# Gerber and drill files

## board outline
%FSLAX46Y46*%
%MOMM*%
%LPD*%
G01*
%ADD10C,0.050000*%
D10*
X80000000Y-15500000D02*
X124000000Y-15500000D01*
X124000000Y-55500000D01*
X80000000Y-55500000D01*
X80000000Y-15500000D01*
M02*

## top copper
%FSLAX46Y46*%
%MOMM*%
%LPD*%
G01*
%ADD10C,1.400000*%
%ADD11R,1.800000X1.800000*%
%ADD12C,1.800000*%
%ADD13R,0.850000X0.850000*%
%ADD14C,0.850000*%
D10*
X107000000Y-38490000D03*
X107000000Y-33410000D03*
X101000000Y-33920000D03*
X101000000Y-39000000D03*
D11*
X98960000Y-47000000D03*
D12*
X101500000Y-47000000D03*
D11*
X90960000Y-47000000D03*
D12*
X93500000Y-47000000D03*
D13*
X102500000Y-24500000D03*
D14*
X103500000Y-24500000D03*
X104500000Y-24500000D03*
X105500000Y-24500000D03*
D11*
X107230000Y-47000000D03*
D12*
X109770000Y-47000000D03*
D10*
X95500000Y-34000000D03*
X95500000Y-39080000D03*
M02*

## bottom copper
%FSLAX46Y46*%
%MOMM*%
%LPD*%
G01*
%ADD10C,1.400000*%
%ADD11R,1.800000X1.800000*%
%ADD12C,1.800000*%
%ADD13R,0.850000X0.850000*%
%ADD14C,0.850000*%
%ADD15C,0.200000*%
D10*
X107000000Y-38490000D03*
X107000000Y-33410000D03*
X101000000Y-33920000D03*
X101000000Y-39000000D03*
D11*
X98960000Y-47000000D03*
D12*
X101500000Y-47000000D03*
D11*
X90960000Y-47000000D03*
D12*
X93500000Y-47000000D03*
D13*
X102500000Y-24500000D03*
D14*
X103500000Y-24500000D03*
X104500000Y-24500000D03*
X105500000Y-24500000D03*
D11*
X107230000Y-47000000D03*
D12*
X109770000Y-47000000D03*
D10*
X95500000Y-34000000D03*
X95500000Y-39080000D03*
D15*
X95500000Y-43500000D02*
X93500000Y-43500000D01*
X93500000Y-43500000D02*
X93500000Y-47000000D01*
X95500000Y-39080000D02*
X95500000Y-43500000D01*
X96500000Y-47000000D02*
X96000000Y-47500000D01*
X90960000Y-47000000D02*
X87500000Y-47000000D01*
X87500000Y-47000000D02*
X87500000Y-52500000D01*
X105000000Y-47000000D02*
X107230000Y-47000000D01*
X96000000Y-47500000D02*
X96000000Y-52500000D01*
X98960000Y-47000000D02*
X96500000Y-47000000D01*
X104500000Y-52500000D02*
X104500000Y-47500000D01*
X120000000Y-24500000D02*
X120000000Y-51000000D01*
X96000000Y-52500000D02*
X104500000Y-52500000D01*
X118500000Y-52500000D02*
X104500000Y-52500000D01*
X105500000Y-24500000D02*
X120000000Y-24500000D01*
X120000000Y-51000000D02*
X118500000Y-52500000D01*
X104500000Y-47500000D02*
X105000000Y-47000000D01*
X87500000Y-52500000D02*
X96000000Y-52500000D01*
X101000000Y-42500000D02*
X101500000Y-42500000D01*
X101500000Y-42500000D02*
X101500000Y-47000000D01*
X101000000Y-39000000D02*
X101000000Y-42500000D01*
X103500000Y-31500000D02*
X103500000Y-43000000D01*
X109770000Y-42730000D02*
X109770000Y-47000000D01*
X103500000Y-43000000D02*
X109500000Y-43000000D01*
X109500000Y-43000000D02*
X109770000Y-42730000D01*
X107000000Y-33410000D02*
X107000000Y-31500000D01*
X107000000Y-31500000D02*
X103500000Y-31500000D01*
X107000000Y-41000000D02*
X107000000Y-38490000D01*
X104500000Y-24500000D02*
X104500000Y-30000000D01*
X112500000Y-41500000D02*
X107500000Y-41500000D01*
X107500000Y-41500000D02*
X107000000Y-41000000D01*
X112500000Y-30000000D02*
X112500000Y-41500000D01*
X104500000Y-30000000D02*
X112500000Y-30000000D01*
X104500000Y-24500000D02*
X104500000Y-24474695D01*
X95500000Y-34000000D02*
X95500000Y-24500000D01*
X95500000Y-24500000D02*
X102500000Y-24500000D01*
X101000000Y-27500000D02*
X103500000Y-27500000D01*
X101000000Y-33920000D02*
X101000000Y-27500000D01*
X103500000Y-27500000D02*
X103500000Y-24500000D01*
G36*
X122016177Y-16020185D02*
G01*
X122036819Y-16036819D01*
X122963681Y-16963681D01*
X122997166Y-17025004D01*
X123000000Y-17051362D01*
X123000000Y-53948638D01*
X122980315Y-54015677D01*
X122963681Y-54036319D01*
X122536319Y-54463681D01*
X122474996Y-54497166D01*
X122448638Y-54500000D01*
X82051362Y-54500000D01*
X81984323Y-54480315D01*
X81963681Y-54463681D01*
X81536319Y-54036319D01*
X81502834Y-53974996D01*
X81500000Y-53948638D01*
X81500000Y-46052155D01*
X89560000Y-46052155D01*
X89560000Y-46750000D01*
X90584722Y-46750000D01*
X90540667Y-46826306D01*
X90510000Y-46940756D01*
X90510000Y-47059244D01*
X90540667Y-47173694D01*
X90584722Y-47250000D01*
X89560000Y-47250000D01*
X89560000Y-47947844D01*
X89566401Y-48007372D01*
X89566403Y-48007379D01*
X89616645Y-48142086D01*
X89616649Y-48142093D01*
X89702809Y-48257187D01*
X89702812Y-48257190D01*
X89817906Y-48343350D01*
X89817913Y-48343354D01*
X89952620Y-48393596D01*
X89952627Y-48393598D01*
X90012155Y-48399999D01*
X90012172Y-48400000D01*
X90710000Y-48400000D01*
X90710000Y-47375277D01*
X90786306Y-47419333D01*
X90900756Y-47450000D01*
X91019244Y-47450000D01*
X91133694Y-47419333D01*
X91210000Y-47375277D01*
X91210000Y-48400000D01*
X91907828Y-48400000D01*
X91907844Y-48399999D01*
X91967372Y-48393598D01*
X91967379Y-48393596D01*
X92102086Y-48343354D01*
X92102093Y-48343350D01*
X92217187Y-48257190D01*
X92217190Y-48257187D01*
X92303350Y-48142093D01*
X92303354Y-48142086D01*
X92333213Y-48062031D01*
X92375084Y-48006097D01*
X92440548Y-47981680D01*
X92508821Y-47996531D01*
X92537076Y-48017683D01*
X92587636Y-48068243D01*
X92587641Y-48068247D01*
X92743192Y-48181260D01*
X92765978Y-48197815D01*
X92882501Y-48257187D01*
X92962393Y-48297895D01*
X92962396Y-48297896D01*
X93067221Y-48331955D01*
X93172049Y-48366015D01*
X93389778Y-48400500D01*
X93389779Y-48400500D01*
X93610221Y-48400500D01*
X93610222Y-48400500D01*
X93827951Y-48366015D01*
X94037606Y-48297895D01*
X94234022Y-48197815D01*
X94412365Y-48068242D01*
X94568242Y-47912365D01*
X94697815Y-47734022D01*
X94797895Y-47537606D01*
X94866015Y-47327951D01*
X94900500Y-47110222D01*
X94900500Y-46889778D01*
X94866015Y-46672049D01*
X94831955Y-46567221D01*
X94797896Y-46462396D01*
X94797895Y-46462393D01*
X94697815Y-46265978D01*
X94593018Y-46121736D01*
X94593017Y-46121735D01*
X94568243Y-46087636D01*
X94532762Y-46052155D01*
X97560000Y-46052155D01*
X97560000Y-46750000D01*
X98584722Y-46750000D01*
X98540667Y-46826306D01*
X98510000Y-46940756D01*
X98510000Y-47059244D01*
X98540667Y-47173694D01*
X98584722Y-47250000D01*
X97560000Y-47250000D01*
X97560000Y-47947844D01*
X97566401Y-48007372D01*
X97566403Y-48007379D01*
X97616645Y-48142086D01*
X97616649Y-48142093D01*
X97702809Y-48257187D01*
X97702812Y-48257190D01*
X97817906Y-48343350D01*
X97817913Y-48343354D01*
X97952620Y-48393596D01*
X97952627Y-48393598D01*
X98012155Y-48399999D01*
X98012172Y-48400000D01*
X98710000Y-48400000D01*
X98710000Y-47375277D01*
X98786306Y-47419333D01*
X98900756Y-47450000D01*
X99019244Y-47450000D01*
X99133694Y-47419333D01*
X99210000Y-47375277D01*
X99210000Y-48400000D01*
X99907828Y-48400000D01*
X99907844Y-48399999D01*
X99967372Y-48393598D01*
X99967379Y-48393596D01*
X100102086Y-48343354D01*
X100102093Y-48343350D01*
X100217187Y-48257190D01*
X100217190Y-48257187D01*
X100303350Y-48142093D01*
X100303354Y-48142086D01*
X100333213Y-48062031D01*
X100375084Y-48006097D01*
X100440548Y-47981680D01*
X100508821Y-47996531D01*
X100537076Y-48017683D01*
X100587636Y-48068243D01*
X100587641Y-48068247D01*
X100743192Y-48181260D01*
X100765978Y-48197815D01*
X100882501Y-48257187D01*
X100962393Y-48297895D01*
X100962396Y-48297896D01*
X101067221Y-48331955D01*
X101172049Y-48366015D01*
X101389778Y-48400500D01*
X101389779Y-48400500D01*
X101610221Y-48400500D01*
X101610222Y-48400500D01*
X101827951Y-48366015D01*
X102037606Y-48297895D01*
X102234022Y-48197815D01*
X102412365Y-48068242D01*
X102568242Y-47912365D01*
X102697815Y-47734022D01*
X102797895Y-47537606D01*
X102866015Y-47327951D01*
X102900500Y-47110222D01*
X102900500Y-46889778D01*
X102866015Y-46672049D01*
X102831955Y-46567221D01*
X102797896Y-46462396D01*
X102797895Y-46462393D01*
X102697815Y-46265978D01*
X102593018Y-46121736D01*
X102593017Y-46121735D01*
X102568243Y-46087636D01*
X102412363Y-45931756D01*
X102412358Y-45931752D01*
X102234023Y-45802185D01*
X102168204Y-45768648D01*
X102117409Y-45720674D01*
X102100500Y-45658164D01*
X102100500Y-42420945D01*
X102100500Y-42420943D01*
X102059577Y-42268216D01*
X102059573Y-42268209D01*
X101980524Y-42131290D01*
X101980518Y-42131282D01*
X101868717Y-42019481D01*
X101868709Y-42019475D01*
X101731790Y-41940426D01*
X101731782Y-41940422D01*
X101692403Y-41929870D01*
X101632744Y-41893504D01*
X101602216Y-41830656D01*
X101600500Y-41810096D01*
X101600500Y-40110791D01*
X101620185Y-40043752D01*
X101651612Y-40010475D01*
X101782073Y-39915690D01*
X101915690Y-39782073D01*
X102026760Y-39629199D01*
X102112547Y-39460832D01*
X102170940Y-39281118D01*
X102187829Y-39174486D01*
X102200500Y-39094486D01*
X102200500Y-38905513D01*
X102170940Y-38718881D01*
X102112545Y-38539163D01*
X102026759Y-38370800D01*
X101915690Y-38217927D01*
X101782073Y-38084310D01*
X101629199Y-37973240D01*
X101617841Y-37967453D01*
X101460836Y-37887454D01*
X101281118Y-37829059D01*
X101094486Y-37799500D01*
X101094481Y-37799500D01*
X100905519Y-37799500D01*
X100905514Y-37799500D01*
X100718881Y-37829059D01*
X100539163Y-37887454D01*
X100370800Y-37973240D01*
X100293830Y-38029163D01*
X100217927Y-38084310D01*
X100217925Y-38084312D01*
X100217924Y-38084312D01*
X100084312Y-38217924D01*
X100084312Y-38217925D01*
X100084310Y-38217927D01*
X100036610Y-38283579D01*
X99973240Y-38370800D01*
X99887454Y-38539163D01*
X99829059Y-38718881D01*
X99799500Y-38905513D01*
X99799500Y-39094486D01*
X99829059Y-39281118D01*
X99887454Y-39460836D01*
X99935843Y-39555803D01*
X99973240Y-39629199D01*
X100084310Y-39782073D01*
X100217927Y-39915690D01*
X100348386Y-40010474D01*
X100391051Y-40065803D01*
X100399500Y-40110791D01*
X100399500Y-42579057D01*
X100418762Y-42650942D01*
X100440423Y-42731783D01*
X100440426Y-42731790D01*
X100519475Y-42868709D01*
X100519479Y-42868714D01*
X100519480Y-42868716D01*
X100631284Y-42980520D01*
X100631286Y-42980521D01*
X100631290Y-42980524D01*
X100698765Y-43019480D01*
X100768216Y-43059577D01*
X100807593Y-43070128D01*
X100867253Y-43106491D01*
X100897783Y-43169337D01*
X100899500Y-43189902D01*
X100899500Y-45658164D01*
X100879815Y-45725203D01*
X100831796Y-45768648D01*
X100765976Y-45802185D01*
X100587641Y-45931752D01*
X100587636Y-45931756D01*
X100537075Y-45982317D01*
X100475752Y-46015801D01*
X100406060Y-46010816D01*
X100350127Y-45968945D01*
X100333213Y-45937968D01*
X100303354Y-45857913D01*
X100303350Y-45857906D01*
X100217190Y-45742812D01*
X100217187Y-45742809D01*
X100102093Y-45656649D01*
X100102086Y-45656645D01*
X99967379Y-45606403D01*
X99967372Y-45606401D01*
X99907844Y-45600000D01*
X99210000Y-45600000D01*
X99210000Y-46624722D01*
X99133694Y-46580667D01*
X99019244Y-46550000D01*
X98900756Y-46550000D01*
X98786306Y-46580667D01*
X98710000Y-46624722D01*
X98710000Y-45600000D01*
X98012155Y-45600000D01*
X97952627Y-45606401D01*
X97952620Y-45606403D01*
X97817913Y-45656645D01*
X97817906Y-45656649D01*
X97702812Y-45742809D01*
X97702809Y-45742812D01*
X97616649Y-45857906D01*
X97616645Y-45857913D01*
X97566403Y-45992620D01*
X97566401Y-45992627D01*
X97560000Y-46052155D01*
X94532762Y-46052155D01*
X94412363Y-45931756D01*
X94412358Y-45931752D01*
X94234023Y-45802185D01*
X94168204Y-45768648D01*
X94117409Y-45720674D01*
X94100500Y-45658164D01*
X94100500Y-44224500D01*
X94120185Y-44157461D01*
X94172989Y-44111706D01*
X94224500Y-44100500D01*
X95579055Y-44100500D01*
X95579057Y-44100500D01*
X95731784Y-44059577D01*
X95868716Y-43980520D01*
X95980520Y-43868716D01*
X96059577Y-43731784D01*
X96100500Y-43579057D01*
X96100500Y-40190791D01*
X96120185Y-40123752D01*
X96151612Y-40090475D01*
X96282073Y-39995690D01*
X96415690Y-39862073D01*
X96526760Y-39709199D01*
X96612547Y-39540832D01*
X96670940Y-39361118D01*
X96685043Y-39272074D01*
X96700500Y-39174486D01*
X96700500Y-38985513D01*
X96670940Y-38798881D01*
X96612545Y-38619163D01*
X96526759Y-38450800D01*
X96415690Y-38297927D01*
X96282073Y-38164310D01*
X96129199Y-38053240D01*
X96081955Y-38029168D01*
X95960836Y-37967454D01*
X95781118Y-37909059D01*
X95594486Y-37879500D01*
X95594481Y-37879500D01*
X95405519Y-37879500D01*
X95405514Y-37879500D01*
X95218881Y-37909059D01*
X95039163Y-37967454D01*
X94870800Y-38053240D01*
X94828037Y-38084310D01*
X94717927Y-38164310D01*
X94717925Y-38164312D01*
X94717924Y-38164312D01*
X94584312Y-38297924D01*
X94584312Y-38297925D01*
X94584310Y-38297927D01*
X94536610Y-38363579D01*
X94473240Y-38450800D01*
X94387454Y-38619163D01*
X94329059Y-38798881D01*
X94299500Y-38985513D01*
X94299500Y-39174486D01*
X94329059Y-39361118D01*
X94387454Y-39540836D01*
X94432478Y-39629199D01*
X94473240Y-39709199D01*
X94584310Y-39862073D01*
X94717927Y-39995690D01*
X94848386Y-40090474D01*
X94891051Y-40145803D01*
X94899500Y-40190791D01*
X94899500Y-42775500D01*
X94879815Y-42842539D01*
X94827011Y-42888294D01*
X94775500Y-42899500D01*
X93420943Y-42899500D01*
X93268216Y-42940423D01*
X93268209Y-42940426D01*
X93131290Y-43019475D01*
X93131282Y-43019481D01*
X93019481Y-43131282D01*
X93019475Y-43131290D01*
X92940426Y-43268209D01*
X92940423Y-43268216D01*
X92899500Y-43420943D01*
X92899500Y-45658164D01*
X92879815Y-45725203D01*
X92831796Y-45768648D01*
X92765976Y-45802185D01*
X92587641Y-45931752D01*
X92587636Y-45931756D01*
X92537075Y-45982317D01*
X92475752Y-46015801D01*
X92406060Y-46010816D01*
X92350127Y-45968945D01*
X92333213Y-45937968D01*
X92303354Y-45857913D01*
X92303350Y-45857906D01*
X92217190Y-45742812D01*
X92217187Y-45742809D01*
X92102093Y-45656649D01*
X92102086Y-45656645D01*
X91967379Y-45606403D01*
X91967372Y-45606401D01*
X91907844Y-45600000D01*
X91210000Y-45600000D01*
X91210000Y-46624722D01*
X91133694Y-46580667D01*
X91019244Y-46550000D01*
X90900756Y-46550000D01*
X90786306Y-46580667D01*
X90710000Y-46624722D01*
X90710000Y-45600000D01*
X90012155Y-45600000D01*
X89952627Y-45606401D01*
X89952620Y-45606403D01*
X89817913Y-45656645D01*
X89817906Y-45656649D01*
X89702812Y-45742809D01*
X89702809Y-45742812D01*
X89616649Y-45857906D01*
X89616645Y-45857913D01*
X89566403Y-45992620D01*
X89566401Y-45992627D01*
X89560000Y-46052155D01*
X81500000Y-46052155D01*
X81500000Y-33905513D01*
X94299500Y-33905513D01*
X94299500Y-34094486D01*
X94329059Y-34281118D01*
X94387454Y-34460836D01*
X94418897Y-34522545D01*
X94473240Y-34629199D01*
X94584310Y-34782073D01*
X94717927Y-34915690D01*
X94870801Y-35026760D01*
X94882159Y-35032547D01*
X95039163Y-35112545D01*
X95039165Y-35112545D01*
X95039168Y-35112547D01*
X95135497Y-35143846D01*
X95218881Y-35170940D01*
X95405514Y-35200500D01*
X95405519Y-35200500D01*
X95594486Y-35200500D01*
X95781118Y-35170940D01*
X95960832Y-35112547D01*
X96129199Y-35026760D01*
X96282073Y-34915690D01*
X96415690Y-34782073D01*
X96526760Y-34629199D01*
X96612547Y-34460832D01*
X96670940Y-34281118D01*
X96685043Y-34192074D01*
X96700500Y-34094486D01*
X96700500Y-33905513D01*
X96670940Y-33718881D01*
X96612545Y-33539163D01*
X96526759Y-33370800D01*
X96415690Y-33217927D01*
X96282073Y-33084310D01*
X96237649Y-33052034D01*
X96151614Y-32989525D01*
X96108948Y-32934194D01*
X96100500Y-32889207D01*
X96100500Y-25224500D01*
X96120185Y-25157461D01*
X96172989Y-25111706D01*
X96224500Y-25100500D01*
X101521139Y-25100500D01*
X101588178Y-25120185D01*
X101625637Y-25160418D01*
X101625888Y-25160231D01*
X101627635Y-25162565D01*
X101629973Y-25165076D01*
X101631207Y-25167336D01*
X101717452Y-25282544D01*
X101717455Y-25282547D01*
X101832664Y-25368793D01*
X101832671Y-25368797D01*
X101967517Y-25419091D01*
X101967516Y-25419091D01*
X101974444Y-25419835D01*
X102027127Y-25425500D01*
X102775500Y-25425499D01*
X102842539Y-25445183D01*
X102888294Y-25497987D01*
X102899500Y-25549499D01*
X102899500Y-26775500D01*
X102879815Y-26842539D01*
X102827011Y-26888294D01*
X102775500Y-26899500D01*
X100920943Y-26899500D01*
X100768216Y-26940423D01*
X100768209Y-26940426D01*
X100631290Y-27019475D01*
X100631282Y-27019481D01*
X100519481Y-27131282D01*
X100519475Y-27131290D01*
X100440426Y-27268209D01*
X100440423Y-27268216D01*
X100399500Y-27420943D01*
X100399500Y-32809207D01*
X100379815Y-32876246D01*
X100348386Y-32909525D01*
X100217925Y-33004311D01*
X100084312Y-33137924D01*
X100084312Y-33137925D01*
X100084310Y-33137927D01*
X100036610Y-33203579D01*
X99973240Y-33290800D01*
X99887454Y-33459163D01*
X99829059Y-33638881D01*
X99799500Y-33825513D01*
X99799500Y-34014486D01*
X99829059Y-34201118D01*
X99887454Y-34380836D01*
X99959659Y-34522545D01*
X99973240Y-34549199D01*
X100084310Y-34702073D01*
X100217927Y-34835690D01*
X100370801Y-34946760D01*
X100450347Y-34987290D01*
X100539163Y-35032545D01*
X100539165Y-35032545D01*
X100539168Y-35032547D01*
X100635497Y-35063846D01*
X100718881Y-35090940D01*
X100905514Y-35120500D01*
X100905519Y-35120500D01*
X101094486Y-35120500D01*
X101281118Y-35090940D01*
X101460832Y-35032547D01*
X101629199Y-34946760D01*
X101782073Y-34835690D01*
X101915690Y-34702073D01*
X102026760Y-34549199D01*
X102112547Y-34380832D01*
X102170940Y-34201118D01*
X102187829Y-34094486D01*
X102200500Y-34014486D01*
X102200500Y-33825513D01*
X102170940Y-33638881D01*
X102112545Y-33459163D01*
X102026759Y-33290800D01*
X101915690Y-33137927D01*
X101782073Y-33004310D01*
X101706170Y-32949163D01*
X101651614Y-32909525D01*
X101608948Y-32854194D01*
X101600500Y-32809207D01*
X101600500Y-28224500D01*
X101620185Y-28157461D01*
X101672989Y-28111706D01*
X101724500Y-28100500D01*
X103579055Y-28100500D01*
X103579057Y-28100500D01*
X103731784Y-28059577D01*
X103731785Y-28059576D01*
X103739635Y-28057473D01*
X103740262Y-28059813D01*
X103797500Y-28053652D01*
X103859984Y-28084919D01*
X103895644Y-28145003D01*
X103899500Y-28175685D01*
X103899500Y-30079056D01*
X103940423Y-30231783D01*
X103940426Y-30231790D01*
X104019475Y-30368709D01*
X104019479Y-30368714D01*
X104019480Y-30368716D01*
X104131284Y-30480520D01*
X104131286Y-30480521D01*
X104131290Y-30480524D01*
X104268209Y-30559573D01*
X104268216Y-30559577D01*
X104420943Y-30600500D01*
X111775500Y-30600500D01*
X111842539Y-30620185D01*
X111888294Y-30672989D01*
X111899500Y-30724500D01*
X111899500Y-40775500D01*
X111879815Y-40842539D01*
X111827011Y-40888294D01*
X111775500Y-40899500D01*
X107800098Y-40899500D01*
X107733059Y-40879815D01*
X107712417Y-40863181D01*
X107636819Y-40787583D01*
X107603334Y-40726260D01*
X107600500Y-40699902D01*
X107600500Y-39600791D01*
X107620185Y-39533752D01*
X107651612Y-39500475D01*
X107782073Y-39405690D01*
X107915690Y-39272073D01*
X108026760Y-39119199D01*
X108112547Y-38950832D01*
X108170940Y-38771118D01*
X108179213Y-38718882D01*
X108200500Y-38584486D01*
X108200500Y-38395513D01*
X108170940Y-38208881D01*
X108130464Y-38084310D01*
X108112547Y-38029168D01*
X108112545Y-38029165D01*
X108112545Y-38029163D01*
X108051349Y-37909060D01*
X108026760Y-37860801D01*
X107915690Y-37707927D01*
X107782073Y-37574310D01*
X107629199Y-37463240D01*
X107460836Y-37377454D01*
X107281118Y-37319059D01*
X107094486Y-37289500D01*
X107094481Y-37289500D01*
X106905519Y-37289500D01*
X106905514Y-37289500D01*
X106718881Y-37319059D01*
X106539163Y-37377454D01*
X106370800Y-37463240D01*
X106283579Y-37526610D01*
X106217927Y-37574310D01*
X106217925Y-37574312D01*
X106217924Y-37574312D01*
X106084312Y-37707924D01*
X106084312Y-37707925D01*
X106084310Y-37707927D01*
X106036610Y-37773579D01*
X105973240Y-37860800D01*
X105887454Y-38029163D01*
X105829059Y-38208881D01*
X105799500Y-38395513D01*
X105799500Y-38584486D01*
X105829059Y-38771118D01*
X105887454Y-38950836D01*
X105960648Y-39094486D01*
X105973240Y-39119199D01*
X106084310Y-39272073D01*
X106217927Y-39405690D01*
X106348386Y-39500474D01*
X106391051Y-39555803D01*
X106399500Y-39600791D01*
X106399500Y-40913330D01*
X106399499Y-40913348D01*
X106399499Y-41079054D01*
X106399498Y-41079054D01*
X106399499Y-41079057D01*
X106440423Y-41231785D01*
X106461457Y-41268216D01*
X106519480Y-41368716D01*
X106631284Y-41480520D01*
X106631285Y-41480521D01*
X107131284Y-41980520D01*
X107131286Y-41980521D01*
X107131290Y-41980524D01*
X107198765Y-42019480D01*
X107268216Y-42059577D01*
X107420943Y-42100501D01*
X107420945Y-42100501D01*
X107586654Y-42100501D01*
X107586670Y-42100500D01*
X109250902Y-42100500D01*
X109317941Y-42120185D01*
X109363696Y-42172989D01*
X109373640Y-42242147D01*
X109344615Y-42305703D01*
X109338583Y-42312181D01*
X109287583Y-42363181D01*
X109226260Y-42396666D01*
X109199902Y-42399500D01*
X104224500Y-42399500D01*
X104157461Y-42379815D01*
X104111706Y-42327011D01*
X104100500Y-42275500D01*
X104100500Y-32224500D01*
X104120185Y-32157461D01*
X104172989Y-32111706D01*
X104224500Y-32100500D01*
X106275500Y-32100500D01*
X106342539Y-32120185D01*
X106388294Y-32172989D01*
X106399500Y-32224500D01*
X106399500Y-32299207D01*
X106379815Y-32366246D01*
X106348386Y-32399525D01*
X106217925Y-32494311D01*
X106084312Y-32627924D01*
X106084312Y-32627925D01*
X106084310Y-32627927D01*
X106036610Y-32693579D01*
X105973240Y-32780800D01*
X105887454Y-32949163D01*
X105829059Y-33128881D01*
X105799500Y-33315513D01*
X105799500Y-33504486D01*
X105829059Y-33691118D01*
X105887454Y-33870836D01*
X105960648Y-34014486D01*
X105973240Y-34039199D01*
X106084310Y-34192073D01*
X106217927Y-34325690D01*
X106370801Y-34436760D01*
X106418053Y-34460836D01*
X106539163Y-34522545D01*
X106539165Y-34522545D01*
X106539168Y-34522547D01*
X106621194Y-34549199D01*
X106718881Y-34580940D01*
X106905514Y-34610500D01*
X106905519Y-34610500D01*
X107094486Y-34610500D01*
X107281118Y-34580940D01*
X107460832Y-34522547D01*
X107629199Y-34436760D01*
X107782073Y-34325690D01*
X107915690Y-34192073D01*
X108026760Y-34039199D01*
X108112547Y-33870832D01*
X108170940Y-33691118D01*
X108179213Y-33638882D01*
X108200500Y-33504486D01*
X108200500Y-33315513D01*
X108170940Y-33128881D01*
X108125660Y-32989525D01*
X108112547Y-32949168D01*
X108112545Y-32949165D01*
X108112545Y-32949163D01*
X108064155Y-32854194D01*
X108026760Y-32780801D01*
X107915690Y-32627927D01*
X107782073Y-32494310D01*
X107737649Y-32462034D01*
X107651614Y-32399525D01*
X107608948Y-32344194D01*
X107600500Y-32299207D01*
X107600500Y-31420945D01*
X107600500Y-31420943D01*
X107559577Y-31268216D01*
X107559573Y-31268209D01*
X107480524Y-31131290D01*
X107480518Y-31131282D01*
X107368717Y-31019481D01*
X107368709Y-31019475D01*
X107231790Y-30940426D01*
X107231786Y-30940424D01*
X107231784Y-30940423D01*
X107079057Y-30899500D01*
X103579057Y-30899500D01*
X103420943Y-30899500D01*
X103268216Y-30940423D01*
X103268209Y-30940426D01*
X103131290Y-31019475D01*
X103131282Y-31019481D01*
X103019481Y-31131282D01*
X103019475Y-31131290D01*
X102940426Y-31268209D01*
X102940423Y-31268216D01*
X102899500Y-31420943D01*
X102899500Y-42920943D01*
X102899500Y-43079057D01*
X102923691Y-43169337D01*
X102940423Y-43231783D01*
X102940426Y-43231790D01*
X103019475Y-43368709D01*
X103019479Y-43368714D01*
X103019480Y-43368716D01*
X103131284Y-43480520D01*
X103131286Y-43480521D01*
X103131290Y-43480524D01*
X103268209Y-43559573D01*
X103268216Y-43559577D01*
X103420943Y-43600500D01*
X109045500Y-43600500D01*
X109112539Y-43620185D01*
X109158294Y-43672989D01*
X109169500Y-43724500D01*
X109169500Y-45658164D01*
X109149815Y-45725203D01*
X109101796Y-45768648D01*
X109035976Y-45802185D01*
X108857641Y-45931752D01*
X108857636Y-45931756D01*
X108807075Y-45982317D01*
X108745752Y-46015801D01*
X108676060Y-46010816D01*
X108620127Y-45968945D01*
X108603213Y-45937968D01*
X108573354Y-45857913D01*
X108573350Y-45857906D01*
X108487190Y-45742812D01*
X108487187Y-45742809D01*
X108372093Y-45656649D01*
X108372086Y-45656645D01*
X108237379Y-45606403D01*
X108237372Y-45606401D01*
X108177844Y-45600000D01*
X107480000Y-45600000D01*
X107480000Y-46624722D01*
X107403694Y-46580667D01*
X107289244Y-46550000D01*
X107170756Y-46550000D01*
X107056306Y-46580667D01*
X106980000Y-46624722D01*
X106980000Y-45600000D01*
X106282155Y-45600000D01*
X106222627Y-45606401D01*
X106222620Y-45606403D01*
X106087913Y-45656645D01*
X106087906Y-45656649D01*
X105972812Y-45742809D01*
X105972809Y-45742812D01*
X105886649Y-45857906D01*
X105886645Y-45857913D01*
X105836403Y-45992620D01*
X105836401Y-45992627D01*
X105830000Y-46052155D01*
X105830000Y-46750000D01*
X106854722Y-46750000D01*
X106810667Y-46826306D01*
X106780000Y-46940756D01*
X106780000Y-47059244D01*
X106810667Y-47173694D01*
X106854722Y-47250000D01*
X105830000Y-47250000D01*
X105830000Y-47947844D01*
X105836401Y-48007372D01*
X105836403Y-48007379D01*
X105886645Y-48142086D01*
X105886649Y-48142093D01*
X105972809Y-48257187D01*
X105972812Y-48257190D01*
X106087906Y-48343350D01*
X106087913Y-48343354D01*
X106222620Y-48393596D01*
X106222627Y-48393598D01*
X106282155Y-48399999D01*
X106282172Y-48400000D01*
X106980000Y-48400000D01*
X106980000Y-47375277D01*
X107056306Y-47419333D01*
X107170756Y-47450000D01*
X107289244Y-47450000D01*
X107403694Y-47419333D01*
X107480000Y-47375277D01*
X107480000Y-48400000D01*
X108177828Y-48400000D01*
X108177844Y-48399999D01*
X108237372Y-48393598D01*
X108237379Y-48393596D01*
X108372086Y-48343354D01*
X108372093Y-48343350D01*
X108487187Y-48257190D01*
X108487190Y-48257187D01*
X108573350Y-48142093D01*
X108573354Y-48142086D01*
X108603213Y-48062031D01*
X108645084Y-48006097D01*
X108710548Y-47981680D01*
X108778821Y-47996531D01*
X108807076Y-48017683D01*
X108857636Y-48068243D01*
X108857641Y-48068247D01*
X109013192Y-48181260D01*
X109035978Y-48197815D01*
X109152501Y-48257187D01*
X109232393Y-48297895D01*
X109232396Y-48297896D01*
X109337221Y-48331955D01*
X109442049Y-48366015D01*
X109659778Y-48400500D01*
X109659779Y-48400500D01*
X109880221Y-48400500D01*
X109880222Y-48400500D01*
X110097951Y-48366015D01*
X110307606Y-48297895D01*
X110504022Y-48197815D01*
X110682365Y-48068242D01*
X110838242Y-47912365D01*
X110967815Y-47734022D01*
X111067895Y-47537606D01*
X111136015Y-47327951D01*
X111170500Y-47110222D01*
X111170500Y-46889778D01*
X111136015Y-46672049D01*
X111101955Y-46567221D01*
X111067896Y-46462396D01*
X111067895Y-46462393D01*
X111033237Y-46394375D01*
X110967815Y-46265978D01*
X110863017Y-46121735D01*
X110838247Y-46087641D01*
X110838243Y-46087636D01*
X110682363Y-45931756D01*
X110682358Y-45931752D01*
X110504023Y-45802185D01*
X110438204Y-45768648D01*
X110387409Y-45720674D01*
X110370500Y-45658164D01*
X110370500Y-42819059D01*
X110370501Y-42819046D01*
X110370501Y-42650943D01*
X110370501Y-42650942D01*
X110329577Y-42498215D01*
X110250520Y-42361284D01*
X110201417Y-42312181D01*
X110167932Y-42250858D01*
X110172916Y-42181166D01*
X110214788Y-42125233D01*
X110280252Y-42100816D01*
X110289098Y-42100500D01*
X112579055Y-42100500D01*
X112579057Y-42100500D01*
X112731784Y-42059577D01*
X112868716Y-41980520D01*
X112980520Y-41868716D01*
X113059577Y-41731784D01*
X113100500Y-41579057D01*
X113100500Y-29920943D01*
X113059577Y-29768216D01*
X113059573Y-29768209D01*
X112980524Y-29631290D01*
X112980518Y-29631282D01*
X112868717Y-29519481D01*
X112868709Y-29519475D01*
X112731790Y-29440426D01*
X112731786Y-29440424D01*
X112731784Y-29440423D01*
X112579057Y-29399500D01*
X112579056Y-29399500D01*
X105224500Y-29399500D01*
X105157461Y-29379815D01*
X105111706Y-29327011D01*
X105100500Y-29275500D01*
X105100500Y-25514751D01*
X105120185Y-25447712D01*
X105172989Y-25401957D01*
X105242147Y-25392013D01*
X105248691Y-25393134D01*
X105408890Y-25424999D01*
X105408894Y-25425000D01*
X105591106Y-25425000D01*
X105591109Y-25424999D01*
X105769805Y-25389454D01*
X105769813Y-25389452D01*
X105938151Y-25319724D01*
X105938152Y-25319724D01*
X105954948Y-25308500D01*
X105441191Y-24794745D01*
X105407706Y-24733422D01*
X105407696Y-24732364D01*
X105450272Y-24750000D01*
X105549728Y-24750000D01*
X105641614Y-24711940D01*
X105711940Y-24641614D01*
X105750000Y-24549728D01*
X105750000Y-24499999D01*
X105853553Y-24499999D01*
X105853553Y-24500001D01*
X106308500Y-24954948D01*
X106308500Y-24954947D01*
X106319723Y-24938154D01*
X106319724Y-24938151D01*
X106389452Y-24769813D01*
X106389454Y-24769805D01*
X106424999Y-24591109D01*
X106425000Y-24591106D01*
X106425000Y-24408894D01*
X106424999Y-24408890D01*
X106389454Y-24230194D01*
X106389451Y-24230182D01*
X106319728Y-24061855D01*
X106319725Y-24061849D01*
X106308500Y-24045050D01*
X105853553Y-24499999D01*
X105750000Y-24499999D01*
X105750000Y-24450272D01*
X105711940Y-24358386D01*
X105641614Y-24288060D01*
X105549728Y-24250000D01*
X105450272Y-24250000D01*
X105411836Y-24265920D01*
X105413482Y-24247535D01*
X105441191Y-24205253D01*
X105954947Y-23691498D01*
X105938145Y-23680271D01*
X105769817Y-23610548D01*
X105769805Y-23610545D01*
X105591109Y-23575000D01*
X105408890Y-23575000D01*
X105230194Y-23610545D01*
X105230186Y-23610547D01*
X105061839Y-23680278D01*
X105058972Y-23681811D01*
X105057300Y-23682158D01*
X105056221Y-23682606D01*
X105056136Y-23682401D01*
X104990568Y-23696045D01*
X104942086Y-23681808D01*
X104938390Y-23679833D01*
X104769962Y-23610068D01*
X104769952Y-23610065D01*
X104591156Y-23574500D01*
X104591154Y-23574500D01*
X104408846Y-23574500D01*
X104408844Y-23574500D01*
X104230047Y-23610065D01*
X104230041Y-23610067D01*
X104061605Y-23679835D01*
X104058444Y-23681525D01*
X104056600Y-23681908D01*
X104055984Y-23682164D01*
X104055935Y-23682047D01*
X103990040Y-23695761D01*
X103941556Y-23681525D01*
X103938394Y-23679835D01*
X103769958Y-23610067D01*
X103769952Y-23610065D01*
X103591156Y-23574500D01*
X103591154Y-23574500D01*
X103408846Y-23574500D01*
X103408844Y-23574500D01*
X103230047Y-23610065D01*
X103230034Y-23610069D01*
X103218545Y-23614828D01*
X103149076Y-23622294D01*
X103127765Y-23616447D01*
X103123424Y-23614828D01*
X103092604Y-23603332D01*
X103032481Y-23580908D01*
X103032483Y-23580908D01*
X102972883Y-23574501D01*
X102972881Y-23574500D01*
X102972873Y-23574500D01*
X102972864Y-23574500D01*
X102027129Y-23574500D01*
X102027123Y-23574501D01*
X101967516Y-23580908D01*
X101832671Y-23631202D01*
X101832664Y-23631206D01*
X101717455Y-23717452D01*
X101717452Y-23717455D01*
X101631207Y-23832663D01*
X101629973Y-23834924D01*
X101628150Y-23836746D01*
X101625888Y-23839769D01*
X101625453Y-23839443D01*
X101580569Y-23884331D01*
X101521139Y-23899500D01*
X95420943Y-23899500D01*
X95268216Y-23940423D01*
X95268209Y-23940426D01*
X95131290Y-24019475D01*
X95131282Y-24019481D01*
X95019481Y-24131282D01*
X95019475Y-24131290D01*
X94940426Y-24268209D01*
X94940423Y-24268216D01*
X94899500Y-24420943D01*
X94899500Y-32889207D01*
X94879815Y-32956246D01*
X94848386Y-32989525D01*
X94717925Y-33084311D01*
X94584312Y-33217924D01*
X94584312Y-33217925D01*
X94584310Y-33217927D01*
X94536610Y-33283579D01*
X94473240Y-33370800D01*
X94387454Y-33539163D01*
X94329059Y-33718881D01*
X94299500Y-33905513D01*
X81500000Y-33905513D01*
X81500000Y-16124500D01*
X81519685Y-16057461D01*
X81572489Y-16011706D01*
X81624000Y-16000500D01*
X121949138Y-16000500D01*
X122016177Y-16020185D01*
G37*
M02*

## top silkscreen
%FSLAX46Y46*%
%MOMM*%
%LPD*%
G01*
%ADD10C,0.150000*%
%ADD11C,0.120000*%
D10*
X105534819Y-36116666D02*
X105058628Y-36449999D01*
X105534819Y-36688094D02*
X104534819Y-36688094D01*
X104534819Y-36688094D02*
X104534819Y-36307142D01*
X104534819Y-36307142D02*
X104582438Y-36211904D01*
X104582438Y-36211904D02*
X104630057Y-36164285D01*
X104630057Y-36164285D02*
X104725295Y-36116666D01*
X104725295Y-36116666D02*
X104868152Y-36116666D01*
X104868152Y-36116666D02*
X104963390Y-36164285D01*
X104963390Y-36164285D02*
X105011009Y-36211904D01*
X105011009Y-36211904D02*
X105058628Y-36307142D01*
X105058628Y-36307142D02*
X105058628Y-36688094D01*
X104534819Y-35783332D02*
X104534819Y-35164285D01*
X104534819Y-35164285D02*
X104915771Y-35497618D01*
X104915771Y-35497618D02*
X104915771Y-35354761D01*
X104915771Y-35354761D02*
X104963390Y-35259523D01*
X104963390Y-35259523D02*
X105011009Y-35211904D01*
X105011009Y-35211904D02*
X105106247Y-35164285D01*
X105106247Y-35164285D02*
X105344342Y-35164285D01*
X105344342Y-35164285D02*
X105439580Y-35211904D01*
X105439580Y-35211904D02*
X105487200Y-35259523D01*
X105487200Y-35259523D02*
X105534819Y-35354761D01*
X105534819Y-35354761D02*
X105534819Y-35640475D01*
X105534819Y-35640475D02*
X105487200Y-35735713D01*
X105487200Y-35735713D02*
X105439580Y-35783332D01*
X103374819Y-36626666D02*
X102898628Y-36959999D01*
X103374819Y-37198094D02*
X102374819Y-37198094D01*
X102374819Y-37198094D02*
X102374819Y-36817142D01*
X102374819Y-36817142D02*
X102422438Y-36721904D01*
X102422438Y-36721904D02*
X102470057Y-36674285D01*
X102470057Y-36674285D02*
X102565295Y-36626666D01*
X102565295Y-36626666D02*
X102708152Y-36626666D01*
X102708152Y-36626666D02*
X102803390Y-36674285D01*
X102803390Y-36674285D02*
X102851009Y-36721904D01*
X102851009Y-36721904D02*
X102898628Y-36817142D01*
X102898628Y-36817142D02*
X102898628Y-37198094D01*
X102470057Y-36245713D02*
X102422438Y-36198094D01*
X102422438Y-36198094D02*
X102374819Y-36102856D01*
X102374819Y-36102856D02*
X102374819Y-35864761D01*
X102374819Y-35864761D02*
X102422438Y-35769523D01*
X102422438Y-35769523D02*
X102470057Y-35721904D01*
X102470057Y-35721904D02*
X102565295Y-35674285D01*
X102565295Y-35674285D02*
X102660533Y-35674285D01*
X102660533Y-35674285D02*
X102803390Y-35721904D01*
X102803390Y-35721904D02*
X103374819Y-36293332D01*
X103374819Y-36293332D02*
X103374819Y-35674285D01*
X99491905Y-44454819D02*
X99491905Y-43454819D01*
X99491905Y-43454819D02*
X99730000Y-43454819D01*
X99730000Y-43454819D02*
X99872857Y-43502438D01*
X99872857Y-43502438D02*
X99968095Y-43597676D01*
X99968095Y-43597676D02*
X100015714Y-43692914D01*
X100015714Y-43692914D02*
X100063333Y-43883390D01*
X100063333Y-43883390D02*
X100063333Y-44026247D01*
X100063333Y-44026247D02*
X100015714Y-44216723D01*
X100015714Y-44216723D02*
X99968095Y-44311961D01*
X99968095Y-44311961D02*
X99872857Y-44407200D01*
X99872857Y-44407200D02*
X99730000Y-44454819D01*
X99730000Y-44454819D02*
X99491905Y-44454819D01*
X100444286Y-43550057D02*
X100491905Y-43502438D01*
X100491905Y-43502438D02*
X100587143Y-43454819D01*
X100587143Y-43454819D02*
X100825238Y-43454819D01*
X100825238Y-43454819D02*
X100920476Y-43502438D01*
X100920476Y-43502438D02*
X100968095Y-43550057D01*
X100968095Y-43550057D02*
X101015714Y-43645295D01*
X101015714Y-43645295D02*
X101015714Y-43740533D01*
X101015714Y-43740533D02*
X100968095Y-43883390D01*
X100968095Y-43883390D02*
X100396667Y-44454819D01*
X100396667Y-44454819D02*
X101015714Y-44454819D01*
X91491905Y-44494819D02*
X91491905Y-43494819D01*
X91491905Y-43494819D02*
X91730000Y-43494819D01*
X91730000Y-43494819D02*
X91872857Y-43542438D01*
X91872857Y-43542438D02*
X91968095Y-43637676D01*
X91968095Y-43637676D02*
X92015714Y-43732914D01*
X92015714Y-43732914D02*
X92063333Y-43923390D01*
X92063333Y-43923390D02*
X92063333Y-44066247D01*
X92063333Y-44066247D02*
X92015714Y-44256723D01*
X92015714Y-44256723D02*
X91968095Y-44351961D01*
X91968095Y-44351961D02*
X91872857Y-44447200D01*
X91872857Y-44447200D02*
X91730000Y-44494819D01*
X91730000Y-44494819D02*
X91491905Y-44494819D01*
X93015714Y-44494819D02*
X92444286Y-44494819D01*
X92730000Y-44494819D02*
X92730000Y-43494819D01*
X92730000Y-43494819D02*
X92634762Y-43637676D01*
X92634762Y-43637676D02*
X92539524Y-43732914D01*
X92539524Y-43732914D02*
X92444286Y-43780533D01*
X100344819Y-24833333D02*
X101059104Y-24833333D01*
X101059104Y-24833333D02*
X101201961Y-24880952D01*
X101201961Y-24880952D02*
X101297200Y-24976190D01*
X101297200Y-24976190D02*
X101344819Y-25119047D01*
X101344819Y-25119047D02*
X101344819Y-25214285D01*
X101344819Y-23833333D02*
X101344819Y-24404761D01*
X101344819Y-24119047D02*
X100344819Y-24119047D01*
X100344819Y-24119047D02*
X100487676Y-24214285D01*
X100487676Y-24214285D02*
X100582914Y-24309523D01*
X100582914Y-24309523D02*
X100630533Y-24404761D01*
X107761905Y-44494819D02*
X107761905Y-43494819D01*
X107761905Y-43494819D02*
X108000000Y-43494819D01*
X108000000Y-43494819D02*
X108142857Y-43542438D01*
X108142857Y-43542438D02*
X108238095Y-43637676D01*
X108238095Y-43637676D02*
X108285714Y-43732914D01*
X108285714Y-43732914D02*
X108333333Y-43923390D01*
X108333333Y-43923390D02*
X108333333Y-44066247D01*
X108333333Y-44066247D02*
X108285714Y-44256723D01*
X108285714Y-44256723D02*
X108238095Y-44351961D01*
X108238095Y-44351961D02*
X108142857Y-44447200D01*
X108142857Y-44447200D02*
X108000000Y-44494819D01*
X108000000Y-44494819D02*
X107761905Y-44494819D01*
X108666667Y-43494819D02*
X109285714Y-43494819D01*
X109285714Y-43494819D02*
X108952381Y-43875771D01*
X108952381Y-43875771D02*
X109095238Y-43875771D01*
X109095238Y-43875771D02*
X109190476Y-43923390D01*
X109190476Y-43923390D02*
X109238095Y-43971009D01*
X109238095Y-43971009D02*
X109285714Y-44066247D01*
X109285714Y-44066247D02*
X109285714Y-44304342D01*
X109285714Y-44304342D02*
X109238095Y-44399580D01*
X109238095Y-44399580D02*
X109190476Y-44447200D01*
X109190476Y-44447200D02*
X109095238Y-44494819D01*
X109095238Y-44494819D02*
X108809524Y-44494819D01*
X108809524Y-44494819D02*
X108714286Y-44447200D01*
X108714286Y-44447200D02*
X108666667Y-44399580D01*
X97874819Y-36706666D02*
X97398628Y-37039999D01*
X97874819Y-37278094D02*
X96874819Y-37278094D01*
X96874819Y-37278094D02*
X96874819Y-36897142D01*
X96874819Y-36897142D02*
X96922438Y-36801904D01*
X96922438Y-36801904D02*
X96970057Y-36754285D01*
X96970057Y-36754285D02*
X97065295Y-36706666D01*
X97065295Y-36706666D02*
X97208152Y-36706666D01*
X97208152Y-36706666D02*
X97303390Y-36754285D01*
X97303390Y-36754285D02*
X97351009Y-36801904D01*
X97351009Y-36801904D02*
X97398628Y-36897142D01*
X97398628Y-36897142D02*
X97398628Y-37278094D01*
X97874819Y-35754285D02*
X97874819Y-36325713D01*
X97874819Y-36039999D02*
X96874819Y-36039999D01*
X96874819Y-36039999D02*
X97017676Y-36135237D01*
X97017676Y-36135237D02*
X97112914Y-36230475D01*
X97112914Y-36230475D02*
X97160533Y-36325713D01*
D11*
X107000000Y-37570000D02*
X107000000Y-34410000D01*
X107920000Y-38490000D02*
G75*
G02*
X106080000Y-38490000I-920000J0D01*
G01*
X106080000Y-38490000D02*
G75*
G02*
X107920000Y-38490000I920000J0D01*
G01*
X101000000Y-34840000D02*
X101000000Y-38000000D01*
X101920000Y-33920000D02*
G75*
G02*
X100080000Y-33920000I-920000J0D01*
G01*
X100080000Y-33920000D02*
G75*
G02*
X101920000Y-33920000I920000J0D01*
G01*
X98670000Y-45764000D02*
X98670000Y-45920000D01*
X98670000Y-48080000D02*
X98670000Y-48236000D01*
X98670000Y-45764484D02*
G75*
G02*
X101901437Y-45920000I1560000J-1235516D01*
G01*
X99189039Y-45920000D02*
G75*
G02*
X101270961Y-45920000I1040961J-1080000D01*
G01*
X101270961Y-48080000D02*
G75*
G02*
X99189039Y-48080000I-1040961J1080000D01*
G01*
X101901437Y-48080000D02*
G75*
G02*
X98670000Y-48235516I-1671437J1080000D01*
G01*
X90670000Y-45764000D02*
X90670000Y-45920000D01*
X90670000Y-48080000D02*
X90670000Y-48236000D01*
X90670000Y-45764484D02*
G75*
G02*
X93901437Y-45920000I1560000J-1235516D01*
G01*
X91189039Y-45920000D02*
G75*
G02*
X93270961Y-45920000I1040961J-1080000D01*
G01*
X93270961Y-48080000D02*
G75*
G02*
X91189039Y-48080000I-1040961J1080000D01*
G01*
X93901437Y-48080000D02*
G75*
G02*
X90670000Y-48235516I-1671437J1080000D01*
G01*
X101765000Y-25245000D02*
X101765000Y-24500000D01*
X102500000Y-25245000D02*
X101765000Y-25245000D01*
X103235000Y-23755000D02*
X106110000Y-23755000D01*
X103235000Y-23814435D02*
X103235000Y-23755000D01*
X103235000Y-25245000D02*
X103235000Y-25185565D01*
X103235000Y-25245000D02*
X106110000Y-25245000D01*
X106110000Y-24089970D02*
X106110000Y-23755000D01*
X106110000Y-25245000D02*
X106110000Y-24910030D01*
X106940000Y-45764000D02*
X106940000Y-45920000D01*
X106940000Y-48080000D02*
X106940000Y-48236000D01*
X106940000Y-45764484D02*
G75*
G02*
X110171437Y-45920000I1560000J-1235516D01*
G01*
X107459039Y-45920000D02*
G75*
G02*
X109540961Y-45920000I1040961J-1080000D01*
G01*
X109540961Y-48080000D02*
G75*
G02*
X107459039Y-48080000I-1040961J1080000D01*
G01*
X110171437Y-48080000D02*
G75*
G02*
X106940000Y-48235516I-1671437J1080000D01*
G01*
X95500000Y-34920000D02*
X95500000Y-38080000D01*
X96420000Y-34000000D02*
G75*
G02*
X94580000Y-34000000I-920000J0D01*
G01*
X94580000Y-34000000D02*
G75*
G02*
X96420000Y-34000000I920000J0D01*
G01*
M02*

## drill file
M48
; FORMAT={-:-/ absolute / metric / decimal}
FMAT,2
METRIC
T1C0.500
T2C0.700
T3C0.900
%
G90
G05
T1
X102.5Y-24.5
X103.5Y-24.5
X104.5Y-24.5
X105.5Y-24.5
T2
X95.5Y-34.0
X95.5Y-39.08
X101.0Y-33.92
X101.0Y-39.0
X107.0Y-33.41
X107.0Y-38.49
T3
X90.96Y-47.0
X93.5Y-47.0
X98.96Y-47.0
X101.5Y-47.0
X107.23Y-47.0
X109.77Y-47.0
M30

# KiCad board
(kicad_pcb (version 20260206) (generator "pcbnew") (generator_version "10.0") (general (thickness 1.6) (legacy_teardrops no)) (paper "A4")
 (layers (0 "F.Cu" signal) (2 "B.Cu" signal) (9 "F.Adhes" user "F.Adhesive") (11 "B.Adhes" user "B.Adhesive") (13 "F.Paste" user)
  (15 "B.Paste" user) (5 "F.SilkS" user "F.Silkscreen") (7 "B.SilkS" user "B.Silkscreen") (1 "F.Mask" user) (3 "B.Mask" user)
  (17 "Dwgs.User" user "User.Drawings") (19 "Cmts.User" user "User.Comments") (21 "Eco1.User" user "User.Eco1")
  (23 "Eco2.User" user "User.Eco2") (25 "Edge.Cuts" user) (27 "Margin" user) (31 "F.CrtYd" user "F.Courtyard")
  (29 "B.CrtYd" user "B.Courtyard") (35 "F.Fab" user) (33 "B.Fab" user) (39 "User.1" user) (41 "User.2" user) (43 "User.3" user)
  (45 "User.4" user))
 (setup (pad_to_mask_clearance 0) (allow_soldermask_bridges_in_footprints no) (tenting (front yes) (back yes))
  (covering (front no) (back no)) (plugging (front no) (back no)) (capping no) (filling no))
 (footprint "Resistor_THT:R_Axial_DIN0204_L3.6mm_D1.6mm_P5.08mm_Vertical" (layer "F.Cu") (at 107 38.49 90)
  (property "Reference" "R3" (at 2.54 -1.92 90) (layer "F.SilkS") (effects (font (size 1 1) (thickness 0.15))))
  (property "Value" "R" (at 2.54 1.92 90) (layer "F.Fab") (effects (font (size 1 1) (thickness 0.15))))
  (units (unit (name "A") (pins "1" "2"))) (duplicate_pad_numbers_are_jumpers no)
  (fp_line (start 0.92 0) (end 4.08 0) (stroke (width 0.12) (type solid)) (layer "F.SilkS"))
  (fp_circle (center 0 0) (end 0.92 0) (stroke (width 0.12) (type solid)) (fill no) (layer "F.SilkS"))
  (pad "1" thru_hole circle (at 0 0 90) (size 1.4 1.4) (drill 0.7) (layers "*.Cu" "*.Mask") (remove_unused_layers no) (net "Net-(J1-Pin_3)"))
  (pad "2" thru_hole circle (at 5.08 0 90) (size 1.4 1.4) (drill 0.7) (layers "*.Cu" "*.Mask") (remove_unused_layers no) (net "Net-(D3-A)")))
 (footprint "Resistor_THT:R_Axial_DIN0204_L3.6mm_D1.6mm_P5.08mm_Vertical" (layer "F.Cu") (at 101 33.92 -90)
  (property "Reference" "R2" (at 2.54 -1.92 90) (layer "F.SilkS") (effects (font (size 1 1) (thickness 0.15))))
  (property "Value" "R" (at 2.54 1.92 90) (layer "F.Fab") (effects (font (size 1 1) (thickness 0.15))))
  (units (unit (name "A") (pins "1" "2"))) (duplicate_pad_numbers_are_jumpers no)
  (fp_line (start 0.92 0) (end 4.08 0) (stroke (width 0.12) (type solid)) (layer "F.SilkS"))
  (fp_circle (center 0 0) (end 0.92 0) (stroke (width 0.12) (type solid)) (fill no) (layer "F.SilkS"))
  (pad "1" thru_hole circle (at 0 0 270) (size 1.4 1.4) (drill 0.7) (layers "*.Cu" "*.Mask") (remove_unused_layers no)
   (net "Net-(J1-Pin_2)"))
  (pad "2" thru_hole circle (at 5.08 0 270) (size 1.4 1.4) (drill 0.7) (layers "*.Cu" "*.Mask") (remove_unused_layers no) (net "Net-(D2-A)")))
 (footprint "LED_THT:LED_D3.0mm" (layer "F.Cu") (at 98.96 47)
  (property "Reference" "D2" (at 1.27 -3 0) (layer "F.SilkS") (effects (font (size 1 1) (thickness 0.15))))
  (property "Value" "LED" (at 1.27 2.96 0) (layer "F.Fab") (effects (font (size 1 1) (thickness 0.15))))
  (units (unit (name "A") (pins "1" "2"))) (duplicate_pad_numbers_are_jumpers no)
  (fp_line (start -0.29 -1.236) (end -0.29 -1.08) (stroke (width 0.12) (type solid)) (layer "F.SilkS"))
  (fp_line (start -0.29 1.08) (end -0.29 1.236) (stroke (width 0.12) (type solid)) (layer "F.SilkS"))
  (fp_arc (start -0.29 -1.235516) (mid 1.36566 -1.987699) (end 2.941437 -1.08) (stroke (width 0.12) (type solid)) (layer "F.SilkS"))
  (fp_arc (start 0.229039 -1.08) (mid 1.27 -1.5) (end 2.310961 -1.08) (stroke (width 0.12) (type solid)) (layer "F.SilkS"))
  (fp_arc (start 2.310961 1.08) (mid 1.27 1.5) (end 0.229039 1.08) (stroke (width 0.12) (type solid)) (layer "F.SilkS"))
  (fp_arc (start 2.941437 1.08) (mid 1.36566 1.987699) (end -0.29 1.235516) (stroke (width 0.12) (type solid)) (layer "F.SilkS"))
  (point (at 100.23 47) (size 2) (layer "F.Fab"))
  (pad "1" thru_hole rect (at 0 0) (size 1.8 1.8) (drill 0.9) (layers "*.Cu" "*.Mask") (remove_unused_layers no) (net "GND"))
  (pad "2" thru_hole circle (at 2.54 0) (size 1.8 1.8) (drill 0.9) (layers "*.Cu" "*.Mask") (remove_unused_layers no) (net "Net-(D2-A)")))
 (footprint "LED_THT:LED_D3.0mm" (layer "F.Cu") (at 90.96 47)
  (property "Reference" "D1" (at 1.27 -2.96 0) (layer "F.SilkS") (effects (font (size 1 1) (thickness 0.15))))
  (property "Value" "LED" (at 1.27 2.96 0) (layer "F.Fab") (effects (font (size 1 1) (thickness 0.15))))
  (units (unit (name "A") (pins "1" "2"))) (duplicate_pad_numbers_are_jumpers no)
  (fp_line (start -0.29 -1.236) (end -0.29 -1.08) (stroke (width 0.12) (type solid)) (layer "F.SilkS"))
  (fp_line (start -0.29 1.08) (end -0.29 1.236) (stroke (width 0.12) (type solid)) (layer "F.SilkS"))
  (fp_arc (start -0.29 -1.235516) (mid 1.36566 -1.987699) (end 2.941437 -1.08) (stroke (width 0.12) (type solid)) (layer "F.SilkS"))
  (fp_arc (start 0.229039 -1.08) (mid 1.27 -1.5) (end 2.310961 -1.08) (stroke (width 0.12) (type solid)) (layer "F.SilkS"))
  (fp_arc (start 2.310961 1.08) (mid 1.27 1.5) (end 0.229039 1.08) (stroke (width 0.12) (type solid)) (layer "F.SilkS"))
  (fp_arc (start 2.941437 1.08) (mid 1.36566 1.987699) (end -0.29 1.235516) (stroke (width 0.12) (type solid)) (layer "F.SilkS"))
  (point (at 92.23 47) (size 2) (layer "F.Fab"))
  (pad "1" thru_hole rect (at 0 0) (size 1.8 1.8) (drill 0.9) (layers "*.Cu" "*.Mask") (remove_unused_layers no) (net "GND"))
  (pad "2" thru_hole circle (at 2.54 0) (size 1.8 1.8) (drill 0.9) (layers "*.Cu" "*.Mask") (remove_unused_layers no) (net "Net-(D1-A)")))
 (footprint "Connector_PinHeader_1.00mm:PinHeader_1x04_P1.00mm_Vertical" (layer "F.Cu") (at 102.5 24.5 90)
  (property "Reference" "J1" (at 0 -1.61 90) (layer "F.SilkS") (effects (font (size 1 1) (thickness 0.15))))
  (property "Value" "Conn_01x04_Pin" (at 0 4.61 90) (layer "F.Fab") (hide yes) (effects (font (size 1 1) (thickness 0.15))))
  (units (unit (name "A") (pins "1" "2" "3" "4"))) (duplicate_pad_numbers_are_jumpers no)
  (fp_line (start -0.745 -0.735) (end 0 -0.735) (stroke (width 0.12) (type solid)) (layer "F.SilkS"))
  (fp_line (start -0.745 0) (end -0.745 -0.735) (stroke (width 0.12) (type solid)) (layer "F.SilkS"))
  (fp_line (start 0.745 0.735) (end 0.745 3.61) (stroke (width 0.12) (type solid)) (layer "F.SilkS"))
  (fp_line (start 0.685565 0.735) (end 0.745 0.735) (stroke (width 0.12) (type solid)) (layer "F.SilkS"))
  (fp_line (start -0.745 0.735) (end -0.685565 0.735) (stroke (width 0.12) (type solid)) (layer "F.SilkS"))
  (fp_line (start -0.745 0.735) (end -0.745 3.61) (stroke (width 0.12) (type solid)) (layer "F.SilkS"))
  (fp_line (start 0.41003 3.61) (end 0.745 3.61) (stroke (width 0.12) (type solid)) (layer "F.SilkS"))
  (fp_line (start -0.745 3.61) (end -0.41003 3.61) (stroke (width 0.12) (type solid)) (layer "F.SilkS"))
  (pad "1" thru_hole rect (at 0 0 90) (size 0.85 0.85) (drill 0.5) (layers "*.Cu" "*.Mask") (remove_unused_layers no) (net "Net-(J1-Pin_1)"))
  (pad "2" thru_hole circle (at 0 1 90) (size 0.85 0.85) (drill 0.5) (layers "*.Cu" "*.Mask") (remove_unused_layers no)
   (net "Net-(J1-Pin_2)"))
  (pad "3" thru_hole circle (at 0 2 90) (size 0.85 0.85) (drill 0.5) (layers "*.Cu" "*.Mask") (remove_unused_layers no)
   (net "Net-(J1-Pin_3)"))
  (pad "4" thru_hole circle (at 0 3 90) (size 0.85 0.85) (drill 0.5) (layers "*.Cu" "*.Mask") (remove_unused_layers no) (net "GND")))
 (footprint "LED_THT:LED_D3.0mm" (layer "F.Cu") (at 107.23 47)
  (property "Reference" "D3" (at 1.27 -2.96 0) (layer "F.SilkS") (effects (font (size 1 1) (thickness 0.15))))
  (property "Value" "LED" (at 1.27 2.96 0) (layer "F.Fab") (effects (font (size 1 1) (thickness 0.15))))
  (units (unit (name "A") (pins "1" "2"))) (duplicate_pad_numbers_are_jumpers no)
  (fp_line (start -0.29 -1.236) (end -0.29 -1.08) (stroke (width 0.12) (type solid)) (layer "F.SilkS"))
  (fp_line (start -0.29 1.08) (end -0.29 1.236) (stroke (width 0.12) (type solid)) (layer "F.SilkS"))
  (fp_arc (start -0.29 -1.235516) (mid 1.36566 -1.987699) (end 2.941437 -1.08) (stroke (width 0.12) (type solid)) (layer "F.SilkS"))
  (fp_arc (start 0.229039 -1.08) (mid 1.27 -1.5) (end 2.310961 -1.08) (stroke (width 0.12) (type solid)) (layer "F.SilkS"))
  (fp_arc (start 2.310961 1.08) (mid 1.27 1.5) (end 0.229039 1.08) (stroke (width 0.12) (type solid)) (layer "F.SilkS"))
  (fp_arc (start 2.941437 1.08) (mid 1.36566 1.987699) (end -0.29 1.235516) (stroke (width 0.12) (type solid)) (layer "F.SilkS"))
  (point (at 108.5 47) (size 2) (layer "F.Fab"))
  (pad "1" thru_hole rect (at 0 0) (size 1.8 1.8) (drill 0.9) (layers "*.Cu" "*.Mask") (remove_unused_layers no) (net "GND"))
  (pad "2" thru_hole circle (at 2.54 0) (size 1.8 1.8) (drill 0.9) (layers "*.Cu" "*.Mask") (remove_unused_layers no) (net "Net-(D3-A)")))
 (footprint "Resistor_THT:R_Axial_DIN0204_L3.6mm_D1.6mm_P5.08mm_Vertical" (layer "F.Cu") (at 95.5 34 -90)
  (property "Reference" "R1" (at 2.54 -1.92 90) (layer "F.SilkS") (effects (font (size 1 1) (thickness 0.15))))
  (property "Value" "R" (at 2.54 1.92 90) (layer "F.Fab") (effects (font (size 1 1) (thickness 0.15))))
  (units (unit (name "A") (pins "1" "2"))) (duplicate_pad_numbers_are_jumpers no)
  (fp_line (start 0.92 0) (end 4.08 0) (stroke (width 0.12) (type solid)) (layer "F.SilkS"))
  (fp_circle (center 0 0) (end 0.92 0) (stroke (width 0.12) (type solid)) (fill no) (layer "F.SilkS"))
  (pad "1" thru_hole circle (at 0 0 270) (size 1.4 1.4) (drill 0.7) (layers "*.Cu" "*.Mask") (remove_unused_layers no)
   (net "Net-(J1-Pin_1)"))
  (pad "2" thru_hole circle (at 5.08 0 270) (size 1.4 1.4) (drill 0.7) (layers "*.Cu" "*.Mask") (remove_unused_layers no) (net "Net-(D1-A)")))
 (gr_rect (start 80 15.5) (end 124 55.5) (stroke (width 0.05) (type default)) (fill no) (layer "Edge.Cuts"))
 (segment (start 95.5 43.5) (end 93.5 43.5) (width 0.2) (layer "B.Cu") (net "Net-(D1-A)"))
 (segment (start 93.5 43.5) (end 93.5 47) (width 0.2) (layer "B.Cu") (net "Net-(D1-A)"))
 (segment (start 95.5 39.08) (end 95.5 43.5) (width 0.2) (layer "B.Cu") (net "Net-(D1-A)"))
 (segment (start 96.5 47) (end 96 47.5) (width 0.2) (layer "B.Cu") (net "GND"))
 (segment (start 90.96 47) (end 87.5 47) (width 0.2) (layer "B.Cu") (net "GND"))
 (segment (start 87.5 47) (end 87.5 52.5) (width 0.2) (layer "B.Cu") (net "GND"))
 (segment (start 105 47) (end 107.23 47) (width 0.2) (layer "B.Cu") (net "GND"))
 (segment (start 96 47.5) (end 96 52.5) (width 0.2) (layer "B.Cu") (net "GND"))
 (segment (start 98.96 47) (end 96.5 47) (width 0.2) (layer "B.Cu") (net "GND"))
 (segment (start 104.5 52.5) (end 104.5 47.5) (width 0.2) (layer "B.Cu") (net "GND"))
 (segment (start 120 24.5) (end 120 51) (width 0.2) (layer "B.Cu") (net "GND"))
 (segment (start 96 52.5) (end 104.5 52.5) (width 0.2) (layer "B.Cu") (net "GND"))
 (segment (start 118.5 52.5) (end 104.5 52.5) (width 0.2) (layer "B.Cu") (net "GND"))
 (segment (start 105.5 24.5) (end 120 24.5) (width 0.2) (layer "B.Cu") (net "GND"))
 (segment (start 120 51) (end 118.5 52.5) (width 0.2) (layer "B.Cu") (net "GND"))
 (segment (start 104.5 47.5) (end 105 47) (width 0.2) (layer "B.Cu") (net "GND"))
 (segment (start 87.5 52.5) (end 96 52.5) (width 0.2) (layer "B.Cu") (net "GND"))
 (segment (start 101 42.5) (end 101.5 42.5) (width 0.2) (layer "B.Cu") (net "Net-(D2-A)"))
 (segment (start 101.5 42.5) (end 101.5 47) (width 0.2) (layer "B.Cu") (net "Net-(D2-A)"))
 (segment (start 101 39) (end 101 42.5) (width 0.2) (layer "B.Cu") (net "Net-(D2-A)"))
 (segment (start 103.5 31.5) (end 103.5 43) (width 0.2) (layer "B.Cu") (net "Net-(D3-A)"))
 (segment (start 109.77 42.73) (end 109.77 47) (width 0.2) (layer "B.Cu") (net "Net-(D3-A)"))
 (segment (start 103.5 43) (end 109.5 43) (width 0.2) (layer "B.Cu") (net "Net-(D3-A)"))
 (segment (start 109.5 43) (end 109.77 42.73) (width 0.2) (layer "B.Cu") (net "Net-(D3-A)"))
 (segment (start 107 33.41) (end 107 31.5) (width 0.2) (layer "B.Cu") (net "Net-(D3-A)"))
 (segment (start 107 31.5) (end 103.5 31.5) (width 0.2) (layer "B.Cu") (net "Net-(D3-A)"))
 (segment (start 107 41) (end 107 38.49) (width 0.2) (layer "B.Cu") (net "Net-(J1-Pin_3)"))
 (segment (start 104.5 24.5) (end 104.5 30) (width 0.2) (layer "B.Cu") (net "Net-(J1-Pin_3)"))
 (segment (start 112.5 41.5) (end 107.5 41.5) (width 0.2) (layer "B.Cu") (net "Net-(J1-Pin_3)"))
 (segment (start 107.5 41.5) (end 107 41) (width 0.2) (layer "B.Cu") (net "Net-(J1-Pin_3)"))
 (segment (start 112.5 30) (end 112.5 41.5) (width 0.2) (layer "B.Cu") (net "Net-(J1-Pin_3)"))
 (segment (start 104.5 30) (end 112.5 30) (width 0.2) (layer "B.Cu") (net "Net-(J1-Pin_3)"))
 (segment (start 104.5 24.5) (end 104.5 24.474695) (width 0.2) (layer "B.Cu") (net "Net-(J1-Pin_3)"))
 (segment (start 95.5 34) (end 95.5 24.5) (width 0.2) (layer "B.Cu") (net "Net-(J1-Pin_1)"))
 (segment (start 95.5 24.5) (end 102.5 24.5) (width 0.2) (layer "B.Cu") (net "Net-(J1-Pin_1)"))
 (segment (start 101 27.5) (end 103.5 27.5) (width 0.2) (layer "B.Cu") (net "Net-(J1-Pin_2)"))
 (segment (start 101 33.92) (end 101 27.5) (width 0.2) (layer "B.Cu") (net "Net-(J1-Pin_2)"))
 (segment (start 103.5 27.5) (end 103.5 24.5) (width 0.2) (layer "B.Cu") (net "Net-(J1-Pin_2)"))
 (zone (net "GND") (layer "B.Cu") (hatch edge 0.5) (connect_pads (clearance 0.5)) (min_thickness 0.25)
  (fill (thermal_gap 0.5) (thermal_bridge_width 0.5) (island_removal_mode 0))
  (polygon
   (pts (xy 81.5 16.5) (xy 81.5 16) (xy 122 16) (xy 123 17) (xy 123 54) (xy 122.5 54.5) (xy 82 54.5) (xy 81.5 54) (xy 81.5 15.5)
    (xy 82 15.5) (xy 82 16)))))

